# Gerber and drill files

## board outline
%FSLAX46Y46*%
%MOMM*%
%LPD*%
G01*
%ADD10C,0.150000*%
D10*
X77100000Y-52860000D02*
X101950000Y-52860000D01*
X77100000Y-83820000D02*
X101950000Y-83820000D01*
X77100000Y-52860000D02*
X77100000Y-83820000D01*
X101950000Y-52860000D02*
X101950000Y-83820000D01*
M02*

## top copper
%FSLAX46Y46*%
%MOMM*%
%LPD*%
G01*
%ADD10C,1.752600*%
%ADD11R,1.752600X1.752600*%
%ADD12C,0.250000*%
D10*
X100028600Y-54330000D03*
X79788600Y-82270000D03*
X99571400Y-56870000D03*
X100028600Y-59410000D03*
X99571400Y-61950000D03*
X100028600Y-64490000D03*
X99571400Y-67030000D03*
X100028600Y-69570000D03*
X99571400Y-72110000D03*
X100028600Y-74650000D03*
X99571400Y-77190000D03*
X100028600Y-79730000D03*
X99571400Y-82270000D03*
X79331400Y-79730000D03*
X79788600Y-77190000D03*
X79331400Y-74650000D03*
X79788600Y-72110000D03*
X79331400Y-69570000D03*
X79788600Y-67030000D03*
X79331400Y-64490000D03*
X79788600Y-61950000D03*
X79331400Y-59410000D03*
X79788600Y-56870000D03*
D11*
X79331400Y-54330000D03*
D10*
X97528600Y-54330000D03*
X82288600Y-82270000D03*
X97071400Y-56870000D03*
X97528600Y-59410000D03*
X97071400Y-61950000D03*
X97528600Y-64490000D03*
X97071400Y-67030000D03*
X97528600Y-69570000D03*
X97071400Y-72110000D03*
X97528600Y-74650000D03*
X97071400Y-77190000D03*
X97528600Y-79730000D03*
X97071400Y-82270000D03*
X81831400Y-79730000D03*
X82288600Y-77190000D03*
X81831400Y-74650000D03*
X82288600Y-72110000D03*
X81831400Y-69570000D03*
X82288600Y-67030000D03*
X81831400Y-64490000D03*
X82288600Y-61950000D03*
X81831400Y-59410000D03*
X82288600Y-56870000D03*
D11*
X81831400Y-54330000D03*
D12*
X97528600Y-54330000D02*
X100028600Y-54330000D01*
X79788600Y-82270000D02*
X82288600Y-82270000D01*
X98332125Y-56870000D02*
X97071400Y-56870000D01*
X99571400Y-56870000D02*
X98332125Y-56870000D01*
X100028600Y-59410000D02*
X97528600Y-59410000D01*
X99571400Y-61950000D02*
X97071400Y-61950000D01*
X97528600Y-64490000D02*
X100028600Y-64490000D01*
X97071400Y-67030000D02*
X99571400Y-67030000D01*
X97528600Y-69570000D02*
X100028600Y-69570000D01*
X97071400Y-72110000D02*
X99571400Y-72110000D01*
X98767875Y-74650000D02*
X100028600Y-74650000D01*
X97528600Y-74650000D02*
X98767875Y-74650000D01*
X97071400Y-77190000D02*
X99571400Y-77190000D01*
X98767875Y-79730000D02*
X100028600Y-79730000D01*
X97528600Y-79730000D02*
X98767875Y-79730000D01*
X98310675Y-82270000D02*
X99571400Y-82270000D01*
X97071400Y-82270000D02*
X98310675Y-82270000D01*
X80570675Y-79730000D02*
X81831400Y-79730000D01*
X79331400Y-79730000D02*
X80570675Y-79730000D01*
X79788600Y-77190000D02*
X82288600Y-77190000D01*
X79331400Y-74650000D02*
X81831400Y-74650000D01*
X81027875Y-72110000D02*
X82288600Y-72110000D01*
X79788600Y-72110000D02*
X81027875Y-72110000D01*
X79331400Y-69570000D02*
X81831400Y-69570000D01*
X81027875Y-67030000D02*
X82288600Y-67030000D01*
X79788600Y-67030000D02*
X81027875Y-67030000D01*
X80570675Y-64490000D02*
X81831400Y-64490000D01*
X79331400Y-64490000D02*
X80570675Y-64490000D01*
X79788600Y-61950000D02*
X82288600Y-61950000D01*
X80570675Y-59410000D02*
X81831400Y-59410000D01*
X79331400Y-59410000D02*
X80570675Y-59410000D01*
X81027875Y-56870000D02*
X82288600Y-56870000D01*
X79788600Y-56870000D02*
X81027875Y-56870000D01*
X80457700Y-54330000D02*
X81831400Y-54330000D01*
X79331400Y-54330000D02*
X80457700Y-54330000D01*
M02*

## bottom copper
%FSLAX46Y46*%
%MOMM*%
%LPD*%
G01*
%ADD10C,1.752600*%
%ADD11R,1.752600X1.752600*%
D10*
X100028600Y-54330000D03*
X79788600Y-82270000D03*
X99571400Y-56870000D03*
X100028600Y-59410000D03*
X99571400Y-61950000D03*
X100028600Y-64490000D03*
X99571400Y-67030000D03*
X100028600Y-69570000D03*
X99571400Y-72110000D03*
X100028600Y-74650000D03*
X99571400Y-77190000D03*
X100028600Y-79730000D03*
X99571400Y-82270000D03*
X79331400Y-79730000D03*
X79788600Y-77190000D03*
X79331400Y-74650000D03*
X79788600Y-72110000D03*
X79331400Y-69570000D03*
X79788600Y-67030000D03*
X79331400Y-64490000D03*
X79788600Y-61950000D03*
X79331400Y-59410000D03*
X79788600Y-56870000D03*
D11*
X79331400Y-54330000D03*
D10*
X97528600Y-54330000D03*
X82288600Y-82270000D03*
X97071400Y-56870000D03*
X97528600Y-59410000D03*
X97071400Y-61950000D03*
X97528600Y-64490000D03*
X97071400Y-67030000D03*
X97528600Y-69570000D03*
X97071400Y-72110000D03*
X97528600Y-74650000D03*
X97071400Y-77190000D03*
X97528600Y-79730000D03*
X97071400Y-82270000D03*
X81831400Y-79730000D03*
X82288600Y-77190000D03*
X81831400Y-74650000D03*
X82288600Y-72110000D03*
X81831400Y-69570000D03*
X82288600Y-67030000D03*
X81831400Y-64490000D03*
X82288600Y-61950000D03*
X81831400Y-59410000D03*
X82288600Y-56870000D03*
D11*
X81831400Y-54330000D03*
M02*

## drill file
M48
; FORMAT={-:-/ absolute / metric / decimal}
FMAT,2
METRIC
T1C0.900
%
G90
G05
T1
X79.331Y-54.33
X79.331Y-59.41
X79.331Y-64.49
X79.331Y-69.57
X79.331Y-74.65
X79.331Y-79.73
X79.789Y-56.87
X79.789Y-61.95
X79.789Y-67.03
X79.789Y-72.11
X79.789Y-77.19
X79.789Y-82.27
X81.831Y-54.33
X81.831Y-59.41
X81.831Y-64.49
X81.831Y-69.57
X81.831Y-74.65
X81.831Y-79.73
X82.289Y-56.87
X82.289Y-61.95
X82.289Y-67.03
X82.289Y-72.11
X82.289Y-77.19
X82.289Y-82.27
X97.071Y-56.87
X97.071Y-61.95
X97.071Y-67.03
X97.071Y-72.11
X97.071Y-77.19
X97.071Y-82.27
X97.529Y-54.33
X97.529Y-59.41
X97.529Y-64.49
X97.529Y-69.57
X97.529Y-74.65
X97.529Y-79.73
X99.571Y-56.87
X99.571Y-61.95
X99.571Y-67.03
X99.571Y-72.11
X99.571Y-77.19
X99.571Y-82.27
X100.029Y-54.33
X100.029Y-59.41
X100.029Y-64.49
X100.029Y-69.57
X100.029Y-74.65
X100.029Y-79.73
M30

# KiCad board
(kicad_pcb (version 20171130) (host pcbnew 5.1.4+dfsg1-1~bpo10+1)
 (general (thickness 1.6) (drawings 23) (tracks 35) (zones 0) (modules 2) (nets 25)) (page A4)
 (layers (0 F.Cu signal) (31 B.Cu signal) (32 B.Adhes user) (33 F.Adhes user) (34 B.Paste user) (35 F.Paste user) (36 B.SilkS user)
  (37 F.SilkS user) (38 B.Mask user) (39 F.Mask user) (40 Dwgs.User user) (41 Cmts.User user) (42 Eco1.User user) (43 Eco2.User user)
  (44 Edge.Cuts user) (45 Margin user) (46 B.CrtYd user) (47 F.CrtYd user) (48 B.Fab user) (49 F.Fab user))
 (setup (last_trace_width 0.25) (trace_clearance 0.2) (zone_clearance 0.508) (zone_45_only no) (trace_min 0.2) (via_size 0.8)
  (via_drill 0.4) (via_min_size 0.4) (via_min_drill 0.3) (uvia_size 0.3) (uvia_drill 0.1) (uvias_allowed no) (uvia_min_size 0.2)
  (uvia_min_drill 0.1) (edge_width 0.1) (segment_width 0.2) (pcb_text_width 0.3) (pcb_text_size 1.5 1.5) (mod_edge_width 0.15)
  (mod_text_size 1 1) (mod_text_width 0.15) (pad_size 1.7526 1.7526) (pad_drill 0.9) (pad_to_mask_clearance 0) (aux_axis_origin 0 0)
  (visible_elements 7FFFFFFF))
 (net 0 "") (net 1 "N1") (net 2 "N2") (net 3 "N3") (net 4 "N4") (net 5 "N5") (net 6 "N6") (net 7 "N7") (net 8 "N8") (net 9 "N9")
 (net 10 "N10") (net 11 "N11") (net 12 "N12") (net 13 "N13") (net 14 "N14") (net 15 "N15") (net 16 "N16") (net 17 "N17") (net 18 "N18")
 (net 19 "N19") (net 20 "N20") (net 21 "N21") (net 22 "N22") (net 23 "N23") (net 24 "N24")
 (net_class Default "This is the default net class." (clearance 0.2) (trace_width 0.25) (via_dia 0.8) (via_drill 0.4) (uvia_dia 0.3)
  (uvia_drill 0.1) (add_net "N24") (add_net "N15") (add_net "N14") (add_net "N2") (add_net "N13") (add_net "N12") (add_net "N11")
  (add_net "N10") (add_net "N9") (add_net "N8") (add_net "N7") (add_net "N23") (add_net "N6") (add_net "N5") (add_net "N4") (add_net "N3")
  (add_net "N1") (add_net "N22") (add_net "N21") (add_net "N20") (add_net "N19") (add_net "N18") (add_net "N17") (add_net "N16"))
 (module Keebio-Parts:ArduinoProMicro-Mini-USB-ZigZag (layer F.Cu) (at 89.68 68.3 270)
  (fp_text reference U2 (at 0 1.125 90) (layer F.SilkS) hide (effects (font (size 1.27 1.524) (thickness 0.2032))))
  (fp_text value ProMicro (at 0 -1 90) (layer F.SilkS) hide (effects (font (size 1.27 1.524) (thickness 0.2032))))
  (pad 24 thru_hole circle (at -13.97 -10.3486 270) (size 1.7526 1.7526) (drill 0.9) (layers *.Cu *.SilkS *.Mask) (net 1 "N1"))
  (pad 12 thru_hole circle (at 13.97 9.8914 270) (size 1.7526 1.7526) (drill 0.9) (layers *.Cu *.SilkS *.Mask) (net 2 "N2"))
  (pad 23 thru_hole circle (at -11.43 -9.8914 270) (size 1.7526 1.7526) (drill 0.9) (layers *.Cu *.SilkS *.Mask) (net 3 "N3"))
  (pad 22 thru_hole circle (at -8.89 -10.3486 270) (size 1.7526 1.7526) (drill 0.9) (layers *.Cu *.SilkS *.Mask) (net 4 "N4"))
  (pad 21 thru_hole circle (at -6.35 -9.8914 270) (size 1.7526 1.7526) (drill 0.9) (layers *.Cu *.SilkS *.Mask) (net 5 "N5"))
  (pad 20 thru_hole circle (at -3.81 -10.3486 270) (size 1.7526 1.7526) (drill 0.9) (layers *.Cu *.SilkS *.Mask) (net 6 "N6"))
  (pad 19 thru_hole circle (at -1.27 -9.8914 270) (size 1.7526 1.7526) (drill 0.9) (layers *.Cu *.SilkS *.Mask) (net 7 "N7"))
  (pad 18 thru_hole circle (at 1.27 -10.3486 270) (size 1.7526 1.7526) (drill 0.9) (layers *.Cu *.SilkS *.Mask) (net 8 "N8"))
  (pad 17 thru_hole circle (at 3.81 -9.8914 270) (size 1.7526 1.7526) (drill 0.9) (layers *.Cu *.SilkS *.Mask) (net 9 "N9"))
  (pad 16 thru_hole circle (at 6.35 -10.3486 270) (size 1.7526 1.7526) (drill 0.9) (layers *.Cu *.SilkS *.Mask) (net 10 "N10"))
  (pad 15 thru_hole circle (at 8.89 -9.8914 270) (size 1.7526 1.7526) (drill 0.9) (layers *.Cu *.SilkS *.Mask) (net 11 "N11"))
  (pad 14 thru_hole circle (at 11.43 -10.3486 270) (size 1.7526 1.7526) (drill 0.9) (layers *.Cu *.SilkS *.Mask) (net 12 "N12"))
  (pad 13 thru_hole circle (at 13.97 -9.8914 270) (size 1.7526 1.7526) (drill 0.9) (layers *.Cu *.SilkS *.Mask) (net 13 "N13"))
  (pad 11 thru_hole circle (at 11.43 10.3486 270) (size 1.7526 1.7526) (drill 0.9) (layers *.Cu *.SilkS *.Mask) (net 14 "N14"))
  (pad 10 thru_hole circle (at 8.89 9.8914 270) (size 1.7526 1.7526) (drill 0.9) (layers *.Cu *.SilkS *.Mask) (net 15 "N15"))
  (pad 9 thru_hole circle (at 6.35 10.3486 270) (size 1.7526 1.7526) (drill 0.9) (layers *.Cu *.SilkS *.Mask) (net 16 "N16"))
  (pad 8 thru_hole circle (at 3.81 9.8914 270) (size 1.7526 1.7526) (drill 0.9) (layers *.Cu *.SilkS *.Mask) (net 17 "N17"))
  (pad 7 thru_hole circle (at 1.27 10.3486 270) (size 1.7526 1.7526) (drill 0.9) (layers *.Cu *.SilkS *.Mask) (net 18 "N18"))
  (pad 6 thru_hole circle (at -1.27 9.8914 270) (size 1.7526 1.7526) (drill 0.9) (layers *.Cu *.SilkS *.Mask) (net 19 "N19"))
  (pad 5 thru_hole circle (at -3.81 10.3486 270) (size 1.7526 1.7526) (drill 0.9) (layers *.Cu *.SilkS *.Mask) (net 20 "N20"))
  (pad 4 thru_hole circle (at -6.35 9.8914 270) (size 1.7526 1.7526) (drill 0.9) (layers *.Cu *.SilkS *.Mask) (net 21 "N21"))
  (pad 3 thru_hole circle (at -8.89 10.3486 270) (size 1.7526 1.7526) (drill 0.9) (layers *.Cu *.SilkS *.Mask) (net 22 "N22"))
  (pad 2 thru_hole circle (at -11.43 9.8914 270) (size 1.7526 1.7526) (drill 0.9) (layers *.Cu *.SilkS *.Mask) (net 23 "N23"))
  (pad 1 thru_hole rect (at -13.97 10.3486 270) (size 1.7526 1.7526) (drill 0.9) (layers *.Cu *.SilkS *.Mask) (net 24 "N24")))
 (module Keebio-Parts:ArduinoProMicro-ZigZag (layer F.Cu) (at 89.68 68.3 270)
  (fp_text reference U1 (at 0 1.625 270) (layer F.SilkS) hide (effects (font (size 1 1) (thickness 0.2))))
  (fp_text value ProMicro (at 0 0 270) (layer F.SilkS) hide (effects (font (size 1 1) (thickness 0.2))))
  (pad 24 thru_hole circle (at -13.97 -7.8486 270) (size 1.7526 1.7526) (drill 0.9) (layers *.Cu *.SilkS *.Mask) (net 1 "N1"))
  (pad 12 thru_hole circle (at 13.97 7.3914 270) (size 1.7526 1.7526) (drill 0.9) (layers *.Cu *.SilkS *.Mask) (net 2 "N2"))
  (pad 23 thru_hole circle (at -11.43 -7.3914 270) (size 1.7526 1.7526) (drill 0.9) (layers *.Cu *.SilkS *.Mask) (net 3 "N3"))
  (pad 22 thru_hole circle (at -8.89 -7.8486 270) (size 1.7526 1.7526) (drill 0.9) (layers *.Cu *.SilkS *.Mask) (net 4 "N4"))
  (pad 21 thru_hole circle (at -6.35 -7.3914 270) (size 1.7526 1.7526) (drill 0.9) (layers *.Cu *.SilkS *.Mask) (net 5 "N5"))
  (pad 20 thru_hole circle (at -3.81 -7.8486 270) (size 1.7526 1.7526) (drill 0.9) (layers *.Cu *.SilkS *.Mask) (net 6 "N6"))
  (pad 19 thru_hole circle (at -1.27 -7.3914 270) (size 1.7526 1.7526) (drill 0.9) (layers *.Cu *.SilkS *.Mask) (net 7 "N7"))
  (pad 18 thru_hole circle (at 1.27 -7.8486 270) (size 1.7526 1.7526) (drill 0.9) (layers *.Cu *.SilkS *.Mask) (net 8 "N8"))
  (pad 17 thru_hole circle (at 3.81 -7.3914 270) (size 1.7526 1.7526) (drill 0.9) (layers *.Cu *.SilkS *.Mask) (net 9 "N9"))
  (pad 16 thru_hole circle (at 6.35 -7.8486 270) (size 1.7526 1.7526) (drill 0.9) (layers *.Cu *.SilkS *.Mask) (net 10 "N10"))
  (pad 15 thru_hole circle (at 8.89 -7.3914 270) (size 1.7526 1.7526) (drill 0.9) (layers *.Cu *.SilkS *.Mask) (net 11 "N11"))
  (pad 14 thru_hole circle (at 11.43 -7.8486 270) (size 1.7526 1.7526) (drill 0.9) (layers *.Cu *.SilkS *.Mask) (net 12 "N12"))
  (pad 13 thru_hole circle (at 13.97 -7.3914 270) (size 1.7526 1.7526) (drill 0.9) (layers *.Cu *.SilkS *.Mask) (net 13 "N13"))
  (pad 11 thru_hole circle (at 11.43 7.8486 270) (size 1.7526 1.7526) (drill 0.9) (layers *.Cu *.SilkS *.Mask) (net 14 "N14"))
  (pad 10 thru_hole circle (at 8.89 7.3914 270) (size 1.7526 1.7526) (drill 0.9) (layers *.Cu *.SilkS *.Mask) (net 15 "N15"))
  (pad 9 thru_hole circle (at 6.35 7.8486 270) (size 1.7526 1.7526) (drill 0.9) (layers *.Cu *.SilkS *.Mask) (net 16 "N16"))
  (pad 8 thru_hole circle (at 3.81 7.3914 270) (size 1.7526 1.7526) (drill 0.9) (layers *.Cu *.SilkS *.Mask) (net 17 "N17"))
  (pad 7 thru_hole circle (at 1.27 7.8486 270) (size 1.7526 1.7526) (drill 0.9) (layers *.Cu *.SilkS *.Mask) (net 18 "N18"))
  (pad 6 thru_hole circle (at -1.27 7.3914 270) (size 1.7526 1.7526) (drill 0.9) (layers *.Cu *.SilkS *.Mask) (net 19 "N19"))
  (pad 5 thru_hole circle (at -3.81 7.8486 270) (size 1.7526 1.7526) (drill 0.9) (layers *.Cu *.SilkS *.Mask) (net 20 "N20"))
  (pad 4 thru_hole circle (at -6.35 7.3914 270) (size 1.7526 1.7526) (drill 0.9) (layers *.Cu *.SilkS *.Mask) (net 21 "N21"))
  (pad 3 thru_hole circle (at -8.89 7.8486 270) (size 1.7526 1.7526) (drill 0.9) (layers *.Cu *.SilkS *.Mask) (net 22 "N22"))
  (pad 2 thru_hole circle (at -11.43 7.3914 270) (size 1.7526 1.7526) (drill 0.9) (layers *.Cu *.SilkS *.Mask) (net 23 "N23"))
  (pad 1 thru_hole rect (at -13.97 7.8486 270) (size 1.7526 1.7526) (drill 0.9) (layers *.Cu *.SilkS *.Mask) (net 24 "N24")))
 (gr_line (start 77.1 52.86) (end 101.95 52.86) (layer Edge.Cuts) (width 0.15))
 (gr_line (start 77.1 83.82) (end 101.95 83.82) (layer Edge.Cuts) (width 0.15))
 (gr_line (start 77.1 52.86) (end 77.1 83.82) (layer Edge.Cuts) (width 0.15))
 (gr_line (start 101.95 52.86) (end 101.95 83.82) (layer Edge.Cuts) (width 0.15))
 (segment (start 97.5286 54.33) (end 100.0286 54.33) (width 0.25) (layer F.Cu) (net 1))
 (segment (start 79.7886 82.27) (end 82.2886 82.27) (width 0.25) (layer F.Cu) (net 2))
 (segment (start 98.332125 56.87) (end 97.0714 56.87) (width 0.25) (layer F.Cu) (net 3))
 (segment (start 99.5714 56.87) (end 98.332125 56.87) (width 0.25) (layer F.Cu) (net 3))
 (segment (start 100.0286 59.41) (end 97.5286 59.41) (width 0.25) (layer F.Cu) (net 4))
 (segment (start 99.5714 61.95) (end 97.0714 61.95) (width 0.25) (layer F.Cu) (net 5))
 (segment (start 97.5286 64.49) (end 100.0286 64.49) (width 0.25) (layer F.Cu) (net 6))
 (segment (start 97.0714 67.03) (end 99.5714 67.03) (width 0.25) (layer F.Cu) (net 7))
 (segment (start 97.5286 69.57) (end 100.0286 69.57) (width 0.25) (layer F.Cu) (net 8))
 (segment (start 97.0714 72.11) (end 99.5714 72.11) (width 0.25) (layer F.Cu) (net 9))
 (segment (start 98.767875 74.65) (end 100.0286 74.65) (width 0.25) (layer F.Cu) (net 10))
 (segment (start 97.5286 74.65) (end 98.767875 74.65) (width 0.25) (layer F.Cu) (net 10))
 (segment (start 97.0714 77.19) (end 99.5714 77.19) (width 0.25) (layer F.Cu) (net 11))
 (segment (start 98.767875 79.73) (end 100.0286 79.73) (width 0.25) (layer F.Cu) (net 12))
 (segment (start 97.5286 79.73) (end 98.767875 79.73) (width 0.25) (layer F.Cu) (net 12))
 (segment (start 98.310675 82.27) (end 99.5714 82.27) (width 0.25) (layer F.Cu) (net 13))
 (segment (start 97.0714 82.27) (end 98.310675 82.27) (width 0.25) (layer F.Cu) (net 13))
 (segment (start 80.570675 79.73) (end 81.8314 79.73) (width 0.25) (layer F.Cu) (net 14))
 (segment (start 79.3314 79.73) (end 80.570675 79.73) (width 0.25) (layer F.Cu) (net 14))
 (segment (start 79.7886 77.19) (end 82.2886 77.19) (width 0.25) (layer F.Cu) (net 15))
 (segment (start 79.3314 74.65) (end 81.8314 74.65) (width 0.25) (layer F.Cu) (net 16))
 (segment (start 81.027875 72.11) (end 82.2886 72.11) (width 0.25) (layer F.Cu) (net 17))
 (segment (start 79.7886 72.11) (end 81.027875 72.11) (width 0.25) (layer F.Cu) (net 17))
 (segment (start 79.3314 69.57) (end 81.8314 69.57) (width 0.25) (layer F.Cu) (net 18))
 (segment (start 81.027875 67.03) (end 82.2886 67.03) (width 0.25) (layer F.Cu) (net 19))
 (segment (start 79.7886 67.03) (end 81.027875 67.03) (width 0.25) (layer F.Cu) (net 19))
 (segment (start 80.570675 64.49) (end 81.8314 64.49) (width 0.25) (layer F.Cu) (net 20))
 (segment (start 79.3314 64.49) (end 80.570675 64.49) (width 0.25) (layer F.Cu) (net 20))
 (segment (start 79.7886 61.95) (end 82.2886 61.95) (width 0.25) (layer F.Cu) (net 21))
 (segment (start 80.570675 59.41) (end 81.8314 59.41) (width 0.25) (layer F.Cu) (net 22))
 (segment (start 79.3314 59.41) (end 80.570675 59.41) (width 0.25) (layer F.Cu) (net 22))
 (segment (start 81.027875 56.87) (end 82.2886 56.87) (width 0.25) (layer F.Cu) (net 23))
 (segment (start 79.7886 56.87) (end 81.027875 56.87) (width 0.25) (layer F.Cu) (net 23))
 (segment (start 80.4577 54.33) (end 81.8314 54.33) (width 0.25) (layer F.Cu) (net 24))
 (segment (start 79.3314 54.33) (end 80.4577 54.33) (width 0.25) (layer F.Cu) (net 24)))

